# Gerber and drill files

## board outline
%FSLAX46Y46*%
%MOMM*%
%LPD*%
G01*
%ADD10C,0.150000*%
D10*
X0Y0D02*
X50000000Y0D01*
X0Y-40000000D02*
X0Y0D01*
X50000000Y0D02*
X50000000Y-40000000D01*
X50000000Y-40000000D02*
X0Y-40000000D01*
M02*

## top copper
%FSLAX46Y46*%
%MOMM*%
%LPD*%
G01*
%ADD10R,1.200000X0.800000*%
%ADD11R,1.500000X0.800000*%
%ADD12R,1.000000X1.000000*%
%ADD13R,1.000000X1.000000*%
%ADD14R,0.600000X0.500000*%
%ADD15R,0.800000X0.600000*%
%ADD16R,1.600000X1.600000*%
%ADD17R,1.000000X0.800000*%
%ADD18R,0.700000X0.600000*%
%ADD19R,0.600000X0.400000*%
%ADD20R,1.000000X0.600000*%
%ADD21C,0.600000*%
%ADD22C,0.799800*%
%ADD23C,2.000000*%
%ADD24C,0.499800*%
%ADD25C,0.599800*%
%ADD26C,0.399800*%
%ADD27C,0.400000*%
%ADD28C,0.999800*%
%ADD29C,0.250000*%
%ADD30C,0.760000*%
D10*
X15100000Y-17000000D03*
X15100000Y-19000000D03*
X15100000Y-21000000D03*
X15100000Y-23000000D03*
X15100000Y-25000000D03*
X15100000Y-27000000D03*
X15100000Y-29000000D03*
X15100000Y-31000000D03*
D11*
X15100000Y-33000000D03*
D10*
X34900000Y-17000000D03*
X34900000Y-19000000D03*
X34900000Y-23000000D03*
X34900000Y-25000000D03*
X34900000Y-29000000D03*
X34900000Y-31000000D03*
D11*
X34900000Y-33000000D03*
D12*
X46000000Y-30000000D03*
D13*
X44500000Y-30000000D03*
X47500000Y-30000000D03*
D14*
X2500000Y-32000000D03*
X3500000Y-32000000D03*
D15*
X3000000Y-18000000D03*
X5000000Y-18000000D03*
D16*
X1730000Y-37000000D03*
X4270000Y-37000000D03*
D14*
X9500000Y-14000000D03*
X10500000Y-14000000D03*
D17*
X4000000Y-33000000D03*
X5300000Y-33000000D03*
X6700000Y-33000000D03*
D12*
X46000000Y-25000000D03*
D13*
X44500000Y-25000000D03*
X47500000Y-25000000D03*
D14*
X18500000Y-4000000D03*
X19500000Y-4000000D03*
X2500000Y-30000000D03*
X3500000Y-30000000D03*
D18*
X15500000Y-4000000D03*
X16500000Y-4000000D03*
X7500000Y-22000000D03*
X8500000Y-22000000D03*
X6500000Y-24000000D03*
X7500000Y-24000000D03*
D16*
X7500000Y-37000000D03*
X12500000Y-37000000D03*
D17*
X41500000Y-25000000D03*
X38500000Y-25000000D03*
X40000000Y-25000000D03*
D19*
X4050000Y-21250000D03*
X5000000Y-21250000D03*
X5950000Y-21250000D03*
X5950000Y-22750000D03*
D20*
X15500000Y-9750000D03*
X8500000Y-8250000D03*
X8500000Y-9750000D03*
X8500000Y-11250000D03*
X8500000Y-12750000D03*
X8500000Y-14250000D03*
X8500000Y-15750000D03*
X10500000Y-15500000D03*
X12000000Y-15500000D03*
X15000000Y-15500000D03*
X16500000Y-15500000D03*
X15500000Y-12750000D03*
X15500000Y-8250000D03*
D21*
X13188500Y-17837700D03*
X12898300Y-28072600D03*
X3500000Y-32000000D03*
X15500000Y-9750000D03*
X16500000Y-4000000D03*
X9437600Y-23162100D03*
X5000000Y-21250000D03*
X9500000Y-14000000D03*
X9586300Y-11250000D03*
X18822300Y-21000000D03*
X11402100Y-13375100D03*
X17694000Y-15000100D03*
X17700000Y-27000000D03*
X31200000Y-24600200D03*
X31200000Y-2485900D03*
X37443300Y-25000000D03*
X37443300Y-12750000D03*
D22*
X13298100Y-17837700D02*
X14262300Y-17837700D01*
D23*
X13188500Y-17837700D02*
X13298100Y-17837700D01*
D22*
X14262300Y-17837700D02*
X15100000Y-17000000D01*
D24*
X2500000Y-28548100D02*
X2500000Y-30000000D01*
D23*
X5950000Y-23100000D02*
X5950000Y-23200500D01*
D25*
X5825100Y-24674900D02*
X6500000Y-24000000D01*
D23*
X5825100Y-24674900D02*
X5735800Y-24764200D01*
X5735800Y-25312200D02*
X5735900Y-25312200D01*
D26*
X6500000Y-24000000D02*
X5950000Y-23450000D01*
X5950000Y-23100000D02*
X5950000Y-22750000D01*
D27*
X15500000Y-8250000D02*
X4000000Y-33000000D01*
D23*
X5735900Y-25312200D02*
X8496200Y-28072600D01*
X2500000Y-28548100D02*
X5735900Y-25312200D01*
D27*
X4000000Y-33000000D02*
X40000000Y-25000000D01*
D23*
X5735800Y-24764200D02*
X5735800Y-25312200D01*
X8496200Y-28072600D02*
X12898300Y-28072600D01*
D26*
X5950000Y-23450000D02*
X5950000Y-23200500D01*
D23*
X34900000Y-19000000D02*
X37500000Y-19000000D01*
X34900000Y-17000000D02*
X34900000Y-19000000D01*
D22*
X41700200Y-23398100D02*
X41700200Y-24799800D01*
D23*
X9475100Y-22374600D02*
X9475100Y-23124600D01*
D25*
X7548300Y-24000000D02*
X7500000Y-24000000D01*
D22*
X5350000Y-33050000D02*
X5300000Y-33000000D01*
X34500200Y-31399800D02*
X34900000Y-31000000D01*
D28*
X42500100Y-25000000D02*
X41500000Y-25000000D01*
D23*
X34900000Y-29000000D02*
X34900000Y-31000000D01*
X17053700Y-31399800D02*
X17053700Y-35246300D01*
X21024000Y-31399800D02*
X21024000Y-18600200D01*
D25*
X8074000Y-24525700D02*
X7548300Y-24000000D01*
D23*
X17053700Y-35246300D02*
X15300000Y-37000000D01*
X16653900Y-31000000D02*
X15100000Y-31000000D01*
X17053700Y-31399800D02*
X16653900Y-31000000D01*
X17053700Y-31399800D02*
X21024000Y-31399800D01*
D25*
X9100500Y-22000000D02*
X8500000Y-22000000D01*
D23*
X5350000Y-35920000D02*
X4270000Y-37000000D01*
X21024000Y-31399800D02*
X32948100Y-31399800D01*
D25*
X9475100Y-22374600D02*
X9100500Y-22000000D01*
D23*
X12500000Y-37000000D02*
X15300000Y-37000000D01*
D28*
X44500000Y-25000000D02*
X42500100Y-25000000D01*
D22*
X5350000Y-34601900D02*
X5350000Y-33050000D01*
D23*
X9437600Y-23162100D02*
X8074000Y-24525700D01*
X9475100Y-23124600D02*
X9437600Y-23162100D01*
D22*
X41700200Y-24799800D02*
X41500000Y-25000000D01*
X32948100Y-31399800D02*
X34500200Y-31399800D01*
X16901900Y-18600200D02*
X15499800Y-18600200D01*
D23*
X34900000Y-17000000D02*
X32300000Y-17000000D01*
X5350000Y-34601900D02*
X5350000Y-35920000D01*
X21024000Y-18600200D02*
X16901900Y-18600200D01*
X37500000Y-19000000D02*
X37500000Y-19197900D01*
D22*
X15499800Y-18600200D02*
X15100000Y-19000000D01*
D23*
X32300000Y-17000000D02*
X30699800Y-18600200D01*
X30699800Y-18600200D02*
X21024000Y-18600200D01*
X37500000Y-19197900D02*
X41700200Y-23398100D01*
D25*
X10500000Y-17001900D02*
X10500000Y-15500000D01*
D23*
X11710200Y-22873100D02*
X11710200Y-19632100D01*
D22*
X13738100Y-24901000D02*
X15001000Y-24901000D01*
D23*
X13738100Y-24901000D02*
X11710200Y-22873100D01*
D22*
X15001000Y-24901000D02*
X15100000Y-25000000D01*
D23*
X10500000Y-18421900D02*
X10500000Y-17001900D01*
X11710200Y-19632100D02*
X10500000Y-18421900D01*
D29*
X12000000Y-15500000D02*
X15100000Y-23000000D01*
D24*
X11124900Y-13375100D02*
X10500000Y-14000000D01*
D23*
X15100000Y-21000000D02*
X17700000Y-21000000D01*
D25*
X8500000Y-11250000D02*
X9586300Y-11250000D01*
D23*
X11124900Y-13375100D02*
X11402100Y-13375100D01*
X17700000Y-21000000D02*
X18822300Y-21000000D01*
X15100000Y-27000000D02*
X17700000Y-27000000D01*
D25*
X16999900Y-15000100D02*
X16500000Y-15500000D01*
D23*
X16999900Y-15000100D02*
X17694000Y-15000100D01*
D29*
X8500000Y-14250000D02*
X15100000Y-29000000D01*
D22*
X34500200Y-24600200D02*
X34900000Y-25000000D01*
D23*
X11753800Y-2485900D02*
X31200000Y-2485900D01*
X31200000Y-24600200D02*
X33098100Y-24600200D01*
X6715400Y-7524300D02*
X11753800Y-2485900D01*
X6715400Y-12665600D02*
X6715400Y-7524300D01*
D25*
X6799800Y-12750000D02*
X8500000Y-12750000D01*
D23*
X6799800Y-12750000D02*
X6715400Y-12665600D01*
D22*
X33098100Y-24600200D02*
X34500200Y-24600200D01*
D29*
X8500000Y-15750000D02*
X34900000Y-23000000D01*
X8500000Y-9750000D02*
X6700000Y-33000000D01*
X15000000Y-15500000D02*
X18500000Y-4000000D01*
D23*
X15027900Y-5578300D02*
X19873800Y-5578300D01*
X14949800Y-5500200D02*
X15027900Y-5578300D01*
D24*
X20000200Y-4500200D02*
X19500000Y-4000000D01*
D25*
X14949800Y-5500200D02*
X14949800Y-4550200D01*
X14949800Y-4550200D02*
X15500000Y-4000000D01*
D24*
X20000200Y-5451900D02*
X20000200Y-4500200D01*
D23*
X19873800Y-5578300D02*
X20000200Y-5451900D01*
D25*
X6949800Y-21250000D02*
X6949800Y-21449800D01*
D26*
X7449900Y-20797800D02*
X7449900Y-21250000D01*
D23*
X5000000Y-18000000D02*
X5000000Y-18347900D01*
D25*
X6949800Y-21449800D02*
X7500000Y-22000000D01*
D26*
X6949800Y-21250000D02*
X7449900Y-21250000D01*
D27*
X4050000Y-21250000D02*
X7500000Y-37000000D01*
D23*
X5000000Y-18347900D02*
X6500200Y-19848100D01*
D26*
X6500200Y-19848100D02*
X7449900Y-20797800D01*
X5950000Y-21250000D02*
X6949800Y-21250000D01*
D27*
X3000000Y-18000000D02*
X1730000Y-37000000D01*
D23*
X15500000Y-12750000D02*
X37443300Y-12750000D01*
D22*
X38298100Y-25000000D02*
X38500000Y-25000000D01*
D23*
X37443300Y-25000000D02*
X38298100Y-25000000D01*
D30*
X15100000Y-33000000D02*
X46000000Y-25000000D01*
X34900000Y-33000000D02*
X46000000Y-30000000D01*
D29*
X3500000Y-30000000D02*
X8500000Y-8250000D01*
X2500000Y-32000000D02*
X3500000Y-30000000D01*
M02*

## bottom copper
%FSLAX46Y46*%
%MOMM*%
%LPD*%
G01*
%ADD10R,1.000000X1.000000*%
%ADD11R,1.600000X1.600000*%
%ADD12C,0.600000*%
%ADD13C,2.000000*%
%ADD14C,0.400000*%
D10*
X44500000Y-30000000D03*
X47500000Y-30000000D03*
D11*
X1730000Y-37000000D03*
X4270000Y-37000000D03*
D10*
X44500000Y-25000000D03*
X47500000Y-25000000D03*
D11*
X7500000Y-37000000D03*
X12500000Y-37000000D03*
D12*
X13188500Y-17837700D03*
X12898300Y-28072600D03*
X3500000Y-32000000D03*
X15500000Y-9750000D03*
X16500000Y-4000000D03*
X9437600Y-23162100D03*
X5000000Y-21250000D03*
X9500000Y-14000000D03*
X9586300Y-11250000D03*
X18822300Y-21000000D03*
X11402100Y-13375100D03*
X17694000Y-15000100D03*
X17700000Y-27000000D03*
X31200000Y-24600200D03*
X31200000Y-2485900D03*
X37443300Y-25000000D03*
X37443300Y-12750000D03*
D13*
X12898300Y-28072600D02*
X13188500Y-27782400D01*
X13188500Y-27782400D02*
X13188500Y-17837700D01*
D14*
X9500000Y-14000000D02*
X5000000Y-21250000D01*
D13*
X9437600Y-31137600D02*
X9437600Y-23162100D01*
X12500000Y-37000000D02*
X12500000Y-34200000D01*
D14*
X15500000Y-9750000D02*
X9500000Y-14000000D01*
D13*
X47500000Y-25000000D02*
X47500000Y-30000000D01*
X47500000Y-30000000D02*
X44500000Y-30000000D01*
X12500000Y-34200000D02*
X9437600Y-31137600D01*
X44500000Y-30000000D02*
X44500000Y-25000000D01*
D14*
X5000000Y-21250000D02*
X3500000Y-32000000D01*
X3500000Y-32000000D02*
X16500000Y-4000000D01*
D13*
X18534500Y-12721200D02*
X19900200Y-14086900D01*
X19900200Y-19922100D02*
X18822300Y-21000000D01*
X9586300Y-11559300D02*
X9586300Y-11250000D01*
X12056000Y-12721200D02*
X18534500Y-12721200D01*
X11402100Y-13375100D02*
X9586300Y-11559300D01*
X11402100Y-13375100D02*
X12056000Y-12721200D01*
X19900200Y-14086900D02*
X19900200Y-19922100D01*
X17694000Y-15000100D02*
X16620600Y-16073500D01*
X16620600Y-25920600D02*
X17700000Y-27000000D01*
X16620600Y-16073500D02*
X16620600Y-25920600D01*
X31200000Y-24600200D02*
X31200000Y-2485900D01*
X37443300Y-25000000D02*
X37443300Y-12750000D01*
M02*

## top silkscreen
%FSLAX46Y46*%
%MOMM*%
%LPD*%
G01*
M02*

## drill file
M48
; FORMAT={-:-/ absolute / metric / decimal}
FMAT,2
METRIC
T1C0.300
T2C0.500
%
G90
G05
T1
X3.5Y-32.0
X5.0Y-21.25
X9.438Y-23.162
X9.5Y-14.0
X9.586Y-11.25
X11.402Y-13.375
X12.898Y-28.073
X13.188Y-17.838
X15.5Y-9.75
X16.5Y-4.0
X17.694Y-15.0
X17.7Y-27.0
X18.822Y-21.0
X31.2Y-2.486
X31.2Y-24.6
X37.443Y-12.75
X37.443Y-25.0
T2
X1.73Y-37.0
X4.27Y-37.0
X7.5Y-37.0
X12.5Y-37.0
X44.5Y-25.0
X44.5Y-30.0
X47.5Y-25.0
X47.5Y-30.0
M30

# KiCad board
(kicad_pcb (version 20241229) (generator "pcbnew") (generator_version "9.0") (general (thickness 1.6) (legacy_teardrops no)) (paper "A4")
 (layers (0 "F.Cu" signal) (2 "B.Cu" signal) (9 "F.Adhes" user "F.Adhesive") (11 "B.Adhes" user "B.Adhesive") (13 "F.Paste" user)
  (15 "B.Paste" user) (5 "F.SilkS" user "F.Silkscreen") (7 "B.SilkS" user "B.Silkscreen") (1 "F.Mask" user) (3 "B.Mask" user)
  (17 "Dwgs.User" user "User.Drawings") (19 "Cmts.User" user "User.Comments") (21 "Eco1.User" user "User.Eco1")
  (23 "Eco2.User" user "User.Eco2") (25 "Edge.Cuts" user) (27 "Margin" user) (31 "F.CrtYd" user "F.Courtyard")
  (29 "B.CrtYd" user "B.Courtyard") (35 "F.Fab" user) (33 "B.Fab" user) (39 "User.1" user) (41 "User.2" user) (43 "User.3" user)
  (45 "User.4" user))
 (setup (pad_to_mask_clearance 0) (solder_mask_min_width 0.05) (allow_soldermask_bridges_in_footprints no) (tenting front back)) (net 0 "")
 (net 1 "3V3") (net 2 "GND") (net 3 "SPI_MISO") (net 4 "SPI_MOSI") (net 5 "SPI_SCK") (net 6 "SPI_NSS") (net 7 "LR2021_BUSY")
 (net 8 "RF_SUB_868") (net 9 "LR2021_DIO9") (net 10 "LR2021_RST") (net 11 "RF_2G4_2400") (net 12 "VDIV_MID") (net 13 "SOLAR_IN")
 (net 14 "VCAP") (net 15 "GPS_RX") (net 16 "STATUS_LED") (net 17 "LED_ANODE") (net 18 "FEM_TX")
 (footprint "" (layer "F.Cu") (at 25 25)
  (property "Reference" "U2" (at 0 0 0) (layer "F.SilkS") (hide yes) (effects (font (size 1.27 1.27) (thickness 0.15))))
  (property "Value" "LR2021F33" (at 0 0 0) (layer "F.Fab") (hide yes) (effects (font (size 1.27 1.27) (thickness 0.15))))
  (pad "1" smd rect (at -9.9 -8) (size 1.2 0.8) (layers "F.Cu" "F.Mask") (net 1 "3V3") (thermal_bridge_angle 45))
  (pad "2" smd rect (at -9.9 -6) (size 1.2 0.8) (layers "F.Cu" "F.Mask") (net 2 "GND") (thermal_bridge_angle 45))
  (pad "3" smd rect (at -9.9 -4) (size 1.2 0.8) (layers "F.Cu" "F.Mask") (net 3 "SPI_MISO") (thermal_bridge_angle 45))
  (pad "4" smd rect (at -9.9 -2) (size 1.2 0.8) (layers "F.Cu" "F.Mask") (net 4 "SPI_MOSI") (thermal_bridge_angle 45))
  (pad "5" smd rect (at -9.9 0) (size 1.2 0.8) (layers "F.Cu" "F.Mask") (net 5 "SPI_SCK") (thermal_bridge_angle 45))
  (pad "6" smd rect (at -9.9 2) (size 1.2 0.8) (layers "F.Cu" "F.Mask") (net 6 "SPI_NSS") (thermal_bridge_angle 45))
  (pad "7" smd rect (at -9.9 4) (size 1.2 0.8) (layers "F.Cu" "F.Mask") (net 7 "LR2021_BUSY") (thermal_bridge_angle 45))
  (pad "8" smd rect (at -9.9 6) (size 1.2 0.8) (layers "F.Cu" "F.Mask") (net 2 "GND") (thermal_bridge_angle 45))
  (pad "9" smd rect (at -9.9 8) (size 1.5 0.8) (layers "F.Cu" "F.Mask") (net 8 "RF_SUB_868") (thermal_bridge_angle 45))
  (pad "10" smd rect (at 9.9 -8) (size 1.2 0.8) (layers "F.Cu" "F.Mask") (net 2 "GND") (thermal_bridge_angle 45))
  (pad "11" smd rect (at 9.9 -6) (size 1.2 0.8) (layers "F.Cu" "F.Mask") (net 2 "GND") (thermal_bridge_angle 45))
  (pad "13" smd rect (at 9.9 -2) (size 1.2 0.8) (layers "F.Cu" "F.Mask") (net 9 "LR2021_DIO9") (thermal_bridge_angle 45))
  (pad "14" smd rect (at 9.9 0) (size 1.2 0.8) (layers "F.Cu" "F.Mask") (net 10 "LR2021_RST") (thermal_bridge_angle 45))
  (pad "16" smd rect (at 9.9 4) (size 1.2 0.8) (layers "F.Cu" "F.Mask") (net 2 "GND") (thermal_bridge_angle 45))
  (pad "17" smd rect (at 9.9 6) (size 1.2 0.8) (layers "F.Cu" "F.Mask") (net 2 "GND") (thermal_bridge_angle 45))
  (pad "18" smd rect (at 9.9 8) (size 1.5 0.8) (layers "F.Cu" "F.Mask") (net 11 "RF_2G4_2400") (thermal_bridge_angle 45)))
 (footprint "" (layer "F.Cu") (at 46 30)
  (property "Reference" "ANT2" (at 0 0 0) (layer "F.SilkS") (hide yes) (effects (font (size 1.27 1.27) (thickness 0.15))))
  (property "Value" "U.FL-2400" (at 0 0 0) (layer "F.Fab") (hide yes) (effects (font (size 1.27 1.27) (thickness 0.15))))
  (pad "1" smd rect (at 0 0) (size 1 1) (layers "F.Cu" "F.Mask") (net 11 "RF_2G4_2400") (thermal_bridge_angle 45))
  (pad "2" thru_hole rect (at -1.5 0) (size 1 1) (drill 0.5) (layers "*.Cu" "*.Mask") (remove_unused_layers no) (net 2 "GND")
   (thermal_bridge_angle 45))
  (pad "3" thru_hole rect (at 1.5 0) (size 1 1) (drill 0.5) (layers "*.Cu" "*.Mask") (remove_unused_layers no) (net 2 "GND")
   (thermal_bridge_angle 45)))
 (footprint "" (layer "F.Cu") (at 3 32)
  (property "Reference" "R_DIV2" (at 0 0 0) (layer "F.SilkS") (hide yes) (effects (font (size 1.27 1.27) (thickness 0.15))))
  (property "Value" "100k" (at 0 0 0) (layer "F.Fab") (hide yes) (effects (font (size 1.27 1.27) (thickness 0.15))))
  (pad "1" smd rect (at -0.5 0) (size 0.6 0.5) (layers "F.Cu" "F.Mask") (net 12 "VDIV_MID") (thermal_bridge_angle 45))
  (pad "2" smd rect (at 0.5 0) (size 0.6 0.5) (layers "F.Cu" "F.Mask") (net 2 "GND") (thermal_bridge_angle 45)))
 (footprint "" (layer "F.Cu") (at 4 18)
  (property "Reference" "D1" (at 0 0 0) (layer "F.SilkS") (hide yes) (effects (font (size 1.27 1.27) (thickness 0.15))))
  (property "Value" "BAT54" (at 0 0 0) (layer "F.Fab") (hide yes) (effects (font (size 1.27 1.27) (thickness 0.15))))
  (pad "A" smd rect (at -1 0) (size 0.8 0.6) (layers "F.Cu" "F.Mask") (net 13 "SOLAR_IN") (thermal_bridge_angle 45))
  (pad "K" smd rect (at 1 0) (size 0.8 0.6) (layers "F.Cu" "F.Mask") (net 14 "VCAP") (thermal_bridge_angle 45)))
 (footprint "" (layer "F.Cu") (at 3 37)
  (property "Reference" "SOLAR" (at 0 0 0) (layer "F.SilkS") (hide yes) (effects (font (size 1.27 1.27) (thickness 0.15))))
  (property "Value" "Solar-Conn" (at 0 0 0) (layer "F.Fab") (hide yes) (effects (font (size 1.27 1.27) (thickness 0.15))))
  (pad "1" thru_hole rect (at -1.27 0) (size 1.6 1.6) (drill 0.5) (layers "*.Cu" "*.Mask") (remove_unused_layers no) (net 13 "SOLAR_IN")
   (thermal_bridge_angle 45))
  (pad "2" thru_hole rect (at 1.27 0) (size 1.6 1.6) (drill 0.5) (layers "*.Cu" "*.Mask") (remove_unused_layers no) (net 2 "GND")
   (thermal_bridge_angle 45)))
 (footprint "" (layer "F.Cu") (at 10 14)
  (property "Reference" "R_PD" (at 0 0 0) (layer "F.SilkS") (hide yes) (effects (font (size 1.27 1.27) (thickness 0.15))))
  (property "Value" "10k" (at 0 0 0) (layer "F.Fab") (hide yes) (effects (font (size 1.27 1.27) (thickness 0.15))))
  (pad "1" smd rect (at -0.5 0) (size 0.6 0.5) (layers "F.Cu" "F.Mask") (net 2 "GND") (thermal_bridge_angle 45))
  (pad "2" smd rect (at 0.5 0) (size 0.6 0.5) (layers "F.Cu" "F.Mask") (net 3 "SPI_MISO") (thermal_bridge_angle 45)))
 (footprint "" (layer "F.Cu") (at 6 33)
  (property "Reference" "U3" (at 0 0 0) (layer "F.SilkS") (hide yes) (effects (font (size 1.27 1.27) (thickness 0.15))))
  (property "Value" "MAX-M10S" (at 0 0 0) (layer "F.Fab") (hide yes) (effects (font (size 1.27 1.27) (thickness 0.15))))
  (pad "1" smd rect (at -2 0) (size 1 0.8) (layers "F.Cu" "F.Mask") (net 1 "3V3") (thermal_bridge_angle 45))
  (pad "2" smd rect (at -0.7 0) (size 1 0.8) (layers "F.Cu" "F.Mask") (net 2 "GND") (thermal_bridge_angle 45))
  (pad "3" smd rect (at 0.7 0) (size 1 0.8) (layers "F.Cu" "F.Mask") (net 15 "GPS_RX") (thermal_bridge_angle 45)))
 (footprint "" (layer "F.Cu") (at 46 25)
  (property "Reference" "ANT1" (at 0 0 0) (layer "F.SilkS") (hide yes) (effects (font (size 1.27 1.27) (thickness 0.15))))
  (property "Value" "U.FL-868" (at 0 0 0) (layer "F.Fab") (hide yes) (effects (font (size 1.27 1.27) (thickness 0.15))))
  (pad "1" smd rect (at 0 0) (size 1 1) (layers "F.Cu" "F.Mask") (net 8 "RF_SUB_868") (thermal_bridge_angle 45))
  (pad "2" thru_hole rect (at -1.5 0) (size 1 1) (drill 0.5) (layers "*.Cu" "*.Mask") (remove_unused_layers no) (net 2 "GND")
   (thermal_bridge_angle 45))
  (pad "3" thru_hole rect (at 1.5 0) (size 1 1) (drill 0.5) (layers "*.Cu" "*.Mask") (remove_unused_layers no) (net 2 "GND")
   (thermal_bridge_angle 45)))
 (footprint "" (layer "F.Cu") (at 19 4)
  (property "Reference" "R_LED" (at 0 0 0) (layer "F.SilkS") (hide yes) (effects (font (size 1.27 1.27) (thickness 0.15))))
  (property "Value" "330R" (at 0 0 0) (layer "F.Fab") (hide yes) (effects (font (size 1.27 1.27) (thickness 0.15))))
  (pad "1" smd rect (at -0.5 0) (size 0.6 0.5) (layers "F.Cu" "F.Mask") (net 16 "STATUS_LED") (thermal_bridge_angle 45))
  (pad "2" smd rect (at 0.5 0) (size 0.6 0.5) (layers "F.Cu" "F.Mask") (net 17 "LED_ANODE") (thermal_bridge_angle 45)))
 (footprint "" (layer "F.Cu") (at 3 30)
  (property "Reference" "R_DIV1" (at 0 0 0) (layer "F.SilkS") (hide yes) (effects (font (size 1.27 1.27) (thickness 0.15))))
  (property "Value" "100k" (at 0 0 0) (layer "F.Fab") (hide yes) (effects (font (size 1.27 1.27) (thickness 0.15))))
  (pad "1" smd rect (at -0.5 0) (size 0.6 0.5) (layers "F.Cu" "F.Mask") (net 1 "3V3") (thermal_bridge_angle 45))
  (pad "2" smd rect (at 0.5 0) (size 0.6 0.5) (layers "F.Cu" "F.Mask") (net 12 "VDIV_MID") (thermal_bridge_angle 45)))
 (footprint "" (layer "F.Cu") (at 16 4)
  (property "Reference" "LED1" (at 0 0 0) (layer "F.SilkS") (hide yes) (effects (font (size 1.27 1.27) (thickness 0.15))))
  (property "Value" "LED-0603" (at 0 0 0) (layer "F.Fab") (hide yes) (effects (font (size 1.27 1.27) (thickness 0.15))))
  (pad "A" smd rect (at -0.5 0) (size 0.7 0.6) (layers "F.Cu" "F.Mask") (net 17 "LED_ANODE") (thermal_bridge_angle 45))
  (pad "K" smd rect (at 0.5 0) (size 0.7 0.6) (layers "F.Cu" "F.Mask") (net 2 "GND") (thermal_bridge_angle 45)))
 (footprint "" (layer "F.Cu") (at 8 22)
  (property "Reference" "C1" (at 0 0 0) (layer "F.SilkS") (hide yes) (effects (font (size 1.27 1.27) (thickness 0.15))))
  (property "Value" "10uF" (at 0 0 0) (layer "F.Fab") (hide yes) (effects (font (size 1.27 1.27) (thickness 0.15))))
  (pad "1" smd rect (at -0.5 0) (size 0.7 0.6) (layers "F.Cu" "F.Mask") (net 14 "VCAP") (thermal_bridge_angle 45))
  (pad "2" smd rect (at 0.5 0) (size 0.7 0.6) (layers "F.Cu" "F.Mask") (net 2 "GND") (thermal_bridge_angle 45)))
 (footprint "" (layer "F.Cu") (at 7 24)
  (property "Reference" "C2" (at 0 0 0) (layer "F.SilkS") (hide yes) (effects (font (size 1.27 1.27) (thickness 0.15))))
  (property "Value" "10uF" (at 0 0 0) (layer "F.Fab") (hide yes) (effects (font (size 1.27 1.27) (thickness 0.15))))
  (pad "1" smd rect (at -0.5 0) (size 0.7 0.6) (layers "F.Cu" "F.Mask") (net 1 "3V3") (thermal_bridge_angle 45))
  (pad "2" smd rect (at 0.5 0) (size 0.7 0.6) (layers "F.Cu" "F.Mask") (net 2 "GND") (thermal_bridge_angle 45)))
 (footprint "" (layer "F.Cu") (at 10 37)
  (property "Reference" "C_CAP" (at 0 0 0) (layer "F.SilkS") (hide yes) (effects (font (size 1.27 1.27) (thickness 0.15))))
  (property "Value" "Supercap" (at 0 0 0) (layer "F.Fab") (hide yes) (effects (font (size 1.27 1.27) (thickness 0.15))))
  (pad "1" thru_hole rect (at -2.5 0) (size 1.6 1.6) (drill 0.5) (layers "*.Cu" "*.Mask") (remove_unused_layers no) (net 14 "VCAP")
   (thermal_bridge_angle 45))
  (pad "2" thru_hole rect (at 2.5 0) (size 1.6 1.6) (drill 0.5) (layers "*.Cu" "*.Mask") (remove_unused_layers no) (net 2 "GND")
   (thermal_bridge_angle 45)))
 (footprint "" (layer "F.Cu") (at 40 25)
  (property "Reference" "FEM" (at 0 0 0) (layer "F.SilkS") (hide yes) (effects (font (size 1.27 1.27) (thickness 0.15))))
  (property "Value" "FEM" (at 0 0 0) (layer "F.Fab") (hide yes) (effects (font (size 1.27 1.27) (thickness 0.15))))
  (pad "GND" smd rect (at 1.5 0) (size 1 0.8) (layers "F.Cu" "F.Mask") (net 2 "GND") (thermal_bridge_angle 45))
  (pad "TX" smd rect (at -1.5 0) (size 1 0.8) (layers "F.Cu" "F.Mask") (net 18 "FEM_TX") (thermal_bridge_angle 45))
  (pad "VCC" smd rect (at 0 0) (size 1 0.8) (layers "F.Cu" "F.Mask") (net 1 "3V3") (thermal_bridge_angle 45)))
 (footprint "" (layer "F.Cu") (at 5 22)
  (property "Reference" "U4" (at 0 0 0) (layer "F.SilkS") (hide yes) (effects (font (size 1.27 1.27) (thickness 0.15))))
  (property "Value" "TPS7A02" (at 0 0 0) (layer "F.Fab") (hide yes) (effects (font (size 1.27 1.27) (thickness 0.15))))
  (pad "1" smd rect (at -0.95 -0.75) (size 0.6 0.4) (layers "F.Cu" "F.Mask") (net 14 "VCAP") (thermal_bridge_angle 45))
  (pad "2" smd rect (at 0 -0.75) (size 0.6 0.4) (layers "F.Cu" "F.Mask") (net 2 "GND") (thermal_bridge_angle 45))
  (pad "3" smd rect (at 0.95 -0.75) (size 0.6 0.4) (layers "F.Cu" "F.Mask") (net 14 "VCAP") (thermal_bridge_angle 45))
  (pad "4" smd rect (at 0.95 0.75) (size 0.6 0.4) (layers "F.Cu" "F.Mask") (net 1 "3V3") (thermal_bridge_angle 45)))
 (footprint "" (layer "F.Cu") (at 12 12)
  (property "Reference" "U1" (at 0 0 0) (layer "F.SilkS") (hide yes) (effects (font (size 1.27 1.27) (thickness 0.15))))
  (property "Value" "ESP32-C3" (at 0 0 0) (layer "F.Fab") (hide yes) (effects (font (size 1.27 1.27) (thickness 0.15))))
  (pad "GND" smd rect (at 3.5 -2.25) (size 1 0.6) (layers "F.Cu" "F.Mask") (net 2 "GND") (thermal_bridge_angle 45))
  (pad "GPIO0" smd rect (at -3.5 -3.75) (size 1 0.6) (layers "F.Cu" "F.Mask") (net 12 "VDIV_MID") (thermal_bridge_angle 45))
  (pad "GPIO1" smd rect (at -3.5 -2.25) (size 1 0.6) (layers "F.Cu" "F.Mask") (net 15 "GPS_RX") (thermal_bridge_angle 45))
  (pad "GPIO2" smd rect (at -3.5 -0.75) (size 1 0.6) (layers "F.Cu" "F.Mask") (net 3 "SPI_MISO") (thermal_bridge_angle 45))
  (pad "GPIO3" smd rect (at -3.5 0.75) (size 1 0.6) (layers "F.Cu" "F.Mask") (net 10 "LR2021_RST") (thermal_bridge_angle 45))
  (pad "GPIO4" smd rect (at -3.5 2.25) (size 1 0.6) (layers "F.Cu" "F.Mask") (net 7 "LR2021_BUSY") (thermal_bridge_angle 45))
  (pad "GPIO5" smd rect (at -3.5 3.75) (size 1 0.6) (layers "F.Cu" "F.Mask") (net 9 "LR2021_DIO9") (thermal_bridge_angle 45))
  (pad "GPIO6" smd rect (at -1.5 3.5) (size 1 0.6) (layers "F.Cu" "F.Mask") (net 5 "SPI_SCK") (thermal_bridge_angle 45))
  (pad "GPIO7" smd rect (at 0 3.5) (size 1 0.6) (layers "F.Cu" "F.Mask") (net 4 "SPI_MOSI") (thermal_bridge_angle 45))
  (pad "GPIO9" smd rect (at 3 3.5) (size 1 0.6) (layers "F.Cu" "F.Mask") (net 16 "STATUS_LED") (thermal_bridge_angle 45))
  (pad "GPIO10" smd rect (at 4.5 3.5) (size 1 0.6) (layers "F.Cu" "F.Mask") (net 6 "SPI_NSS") (thermal_bridge_angle 45))
  (pad "GPIO19" smd rect (at 3.5 0.75) (size 1 0.6) (layers "F.Cu" "F.Mask") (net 18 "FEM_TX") (thermal_bridge_angle 45))
  (pad "VCC" smd rect (at 3.5 -3.75) (size 1 0.6) (layers "F.Cu" "F.Mask") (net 1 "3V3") (thermal_bridge_angle 45)))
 (gr_line (start 0 0) (end 50 0) (stroke (width 0.15) (type default)) (layer "Edge.Cuts"))
 (gr_line (start 0 40) (end 0 0) (stroke (width 0.15) (type default)) (layer "Edge.Cuts"))
 (gr_line (start 50 0) (end 50 40) (stroke (width 0.15) (type default)) (layer "Edge.Cuts"))
 (gr_line (start 50 40) (end 0 40) (stroke (width 0.15) (type default)) (layer "Edge.Cuts"))
 (segment (start 13.2981 17.8377) (end 14.2623 17.8377) (width 0.7998) (layer "F.Cu") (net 1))
 (segment (start 13.1885 17.8377) (end 13.2981 17.8377) (width 2) (layer "F.Cu") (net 1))
 (segment (start 14.2623 17.8377) (end 15.1 17) (width 0.7998) (layer "F.Cu") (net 1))
 (segment (start 2.5 28.5481) (end 2.5 30) (width 0.4998) (layer "F.Cu") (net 1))
 (segment (start 5.95 23.1) (end 5.95 23.2005) (width 2) (layer "F.Cu") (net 1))
 (segment (start 5.8251 24.6749) (end 6.5 24) (width 0.5998) (layer "F.Cu") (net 1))
 (segment (start 5.8251 24.6749) (end 5.7358 24.7642) (width 2) (layer "F.Cu") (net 1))
 (segment (start 5.7358 25.3122) (end 5.7359 25.3122) (width 2) (layer "F.Cu") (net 1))
 (segment (start 6.5 24) (end 5.95 23.45) (width 0.3998) (layer "F.Cu") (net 1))
 (segment (start 5.95 23.1) (end 5.95 22.75) (width 0.3998) (layer "F.Cu") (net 1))
 (segment (start 15.5 8.25) (end 4 33) (width 0.4) (layer "F.Cu") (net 1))
 (segment (start 5.7359 25.3122) (end 8.4962 28.0726) (width 2) (layer "F.Cu") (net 1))
 (segment (start 2.5 28.5481) (end 5.7359 25.3122) (width 2) (layer "F.Cu") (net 1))
 (segment (start 4 33) (end 40 25) (width 0.4) (layer "F.Cu") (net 1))
 (segment (start 5.7358 24.7642) (end 5.7358 25.3122) (width 2) (layer "F.Cu") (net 1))
 (segment (start 8.4962 28.0726) (end 12.8983 28.0726) (width 2) (layer "F.Cu") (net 1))
 (segment (start 5.95 23.45) (end 5.95 23.2005) (width 0.3998) (layer "F.Cu") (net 1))
 (via (at 13.1885 17.8377) (size 0.6) (drill 0.3) (layers "F.Cu" "B.Cu") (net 1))
 (via (at 12.8983 28.0726) (size 0.6) (drill 0.3) (layers "F.Cu" "B.Cu") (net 1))
 (segment (start 12.8983 28.0726) (end 13.1885 27.7824) (width 2) (layer "B.Cu") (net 1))
 (segment (start 13.1885 27.7824) (end 13.1885 17.8377) (width 2) (layer "B.Cu") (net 1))
 (segment (start 34.9 19) (end 37.5 19) (width 2) (layer "F.Cu") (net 2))
 (segment (start 34.9 17) (end 34.9 19) (width 2) (layer "F.Cu") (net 2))
 (segment (start 41.7002 23.3981) (end 41.7002 24.7998) (width 0.7998) (layer "F.Cu") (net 2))
 (segment (start 9.4751 22.3746) (end 9.4751 23.1246) (width 2) (layer "F.Cu") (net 2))
 (segment (start 7.5483 24) (end 7.5 24) (width 0.5998) (layer "F.Cu") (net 2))
 (segment (start 5.35 33.05) (end 5.3 33) (width 0.7998) (layer "F.Cu") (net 2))
 (segment (start 34.5002 31.3998) (end 34.9 31) (width 0.7998) (layer "F.Cu") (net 2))
 (segment (start 42.5001 25) (end 41.5 25) (width 0.9998) (layer "F.Cu") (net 2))
 (segment (start 34.9 29) (end 34.9 31) (width 2) (layer "F.Cu") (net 2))
 (segment (start 17.0537 31.3998) (end 17.0537 35.2463) (width 2) (layer "F.Cu") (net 2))
 (segment (start 21.024 31.3998) (end 21.024 18.6002) (width 2) (layer "F.Cu") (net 2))
 (segment (start 8.074 24.5257) (end 7.5483 24) (width 0.5998) (layer "F.Cu") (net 2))
 (segment (start 17.0537 35.2463) (end 15.3 37) (width 2) (layer "F.Cu") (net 2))
 (segment (start 16.6539 31) (end 15.1 31) (width 2) (layer "F.Cu") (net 2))
 (segment (start 17.0537 31.3998) (end 16.6539 31) (width 2) (layer "F.Cu") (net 2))
 (segment (start 17.0537 31.3998) (end 21.024 31.3998) (width 2) (layer "F.Cu") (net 2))
 (segment (start 9.1005 22) (end 8.5 22) (width 0.5998) (layer "F.Cu") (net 2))
 (segment (start 5.35 35.92) (end 4.27 37) (width 2) (layer "F.Cu") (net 2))
 (segment (start 21.024 31.3998) (end 32.9481 31.3998) (width 2) (layer "F.Cu") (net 2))
 (segment (start 9.4751 22.3746) (end 9.1005 22) (width 0.5998) (layer "F.Cu") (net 2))
 (segment (start 12.5 37) (end 15.3 37) (width 2) (layer "F.Cu") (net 2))
 (segment (start 44.5 25) (end 42.5001 25) (width 0.9998) (layer "F.Cu") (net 2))
 (segment (start 5.35 34.6019) (end 5.35 33.05) (width 0.7998) (layer "F.Cu") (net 2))
 (segment (start 9.4376 23.1621) (end 8.074 24.5257) (width 2) (layer "F.Cu") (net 2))
 (segment (start 9.4751 23.1246) (end 9.4376 23.1621) (width 2) (layer "F.Cu") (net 2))
 (segment (start 41.7002 24.7998) (end 41.5 25) (width 0.7998) (layer "F.Cu") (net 2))
 (segment (start 32.9481 31.3998) (end 34.5002 31.3998) (width 0.7998) (layer "F.Cu") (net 2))
 (segment (start 16.9019 18.6002) (end 15.4998 18.6002) (width 0.7998) (layer "F.Cu") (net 2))
 (segment (start 34.9 17) (end 32.3 17) (width 2) (layer "F.Cu") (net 2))
 (segment (start 5.35 34.6019) (end 5.35 35.92) (width 2) (layer "F.Cu") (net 2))
 (segment (start 21.024 18.6002) (end 16.9019 18.6002) (width 2) (layer "F.Cu") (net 2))
 (segment (start 37.5 19) (end 37.5 19.1979) (width 2) (layer "F.Cu") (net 2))
 (segment (start 15.4998 18.6002) (end 15.1 19) (width 0.7998) (layer "F.Cu") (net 2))
 (segment (start 32.3 17) (end 30.6998 18.6002) (width 2) (layer "F.Cu") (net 2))
 (segment (start 30.6998 18.6002) (end 21.024 18.6002) (width 2) (layer "F.Cu") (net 2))
 (segment (start 37.5 19.1979) (end 41.7002 23.3981) (width 2) (layer "F.Cu") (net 2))
 (via (at 3.5 32) (size 0.6) (drill 0.3) (layers "F.Cu" "B.Cu") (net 2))
 (via (at 15.5 9.75) (size 0.6) (drill 0.3) (layers "F.Cu" "B.Cu") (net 2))
 (via (at 16.5 4) (size 0.6) (drill 0.3) (layers "F.Cu" "B.Cu") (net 2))
 (via (at 9.4376 23.1621) (size 0.6) (drill 0.3) (layers "F.Cu" "B.Cu") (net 2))
 (via (at 5 21.25) (size 0.6) (drill 0.3) (layers "F.Cu" "B.Cu") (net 2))
 (via (at 9.5 14) (size 0.6) (drill 0.3) (layers "F.Cu" "B.Cu") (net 2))
 (segment (start 9.5 14) (end 5 21.25) (width 0.4) (layer "B.Cu") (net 2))
 (segment (start 9.4376 31.1376) (end 9.4376 23.1621) (width 2) (layer "B.Cu") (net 2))
 (segment (start 12.5 37) (end 12.5 34.2) (width 2) (layer "B.Cu") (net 2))
 (segment (start 15.5 9.75) (end 9.5 14) (width 0.4) (layer "B.Cu") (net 2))
 (segment (start 47.5 25) (end 47.5 30) (width 2) (layer "B.Cu") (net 2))
 (segment (start 47.5 30) (end 44.5 30) (width 2) (layer "B.Cu") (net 2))
 (segment (start 12.5 34.2) (end 9.4376 31.1376) (width 2) (layer "B.Cu") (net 2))
 (segment (start 44.5 30) (end 44.5 25) (width 2) (layer "B.Cu") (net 2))
 (segment (start 5 21.25) (end 3.5 32) (width 0.4) (layer "B.Cu") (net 2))
 (segment (start 3.5 32) (end 16.5 4) (width 0.4) (layer "B.Cu") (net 2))
 (segment (start 10.5 17.0019) (end 10.5 15.5) (width 0.5998) (layer "F.Cu") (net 5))
 (segment (start 11.7102 22.8731) (end 11.7102 19.6321) (width 2) (layer "F.Cu") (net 5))
 (segment (start 13.7381 24.901) (end 15.001 24.901) (width 0.7998) (layer "F.Cu") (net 5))
 (segment (start 13.7381 24.901) (end 11.7102 22.8731) (width 2) (layer "F.Cu") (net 5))
 (segment (start 15.001 24.901) (end 15.1 25) (width 0.7998) (layer "F.Cu") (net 5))
 (segment (start 10.5 18.4219) (end 10.5 17.0019) (width 2) (layer "F.Cu") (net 5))
 (segment (start 11.7102 19.6321) (end 10.5 18.4219) (width 2) (layer "F.Cu") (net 5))
 (segment (start 12 15.5) (end 15.1 23) (width 0.25) (layer "F.Cu") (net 4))
 (segment (start 11.1249 13.3751) (end 10.5 14) (width 0.4998) (layer "F.Cu") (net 3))
 (segment (start 15.1 21) (end 17.7 21) (width 2) (layer "F.Cu") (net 3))
 (segment (start 8.5 11.25) (end 9.5863 11.25) (width 0.5998) (layer "F.Cu") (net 3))
 (segment (start 11.1249 13.3751) (end 11.4021 13.3751) (width 2) (layer "F.Cu") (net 3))
 (segment (start 17.7 21) (end 18.8223 21) (width 2) (layer "F.Cu") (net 3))
 (via (at 9.5863 11.25) (size 0.6) (drill 0.3) (layers "F.Cu" "B.Cu") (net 3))
 (via (at 18.8223 21) (size 0.6) (drill 0.3) (layers "F.Cu" "B.Cu") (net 3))
 (via (at 11.4021 13.3751) (size 0.6) (drill 0.3) (layers "F.Cu" "B.Cu") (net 3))
 (segment (start 18.5345 12.7212) (end 19.9002 14.0869) (width 2) (layer "B.Cu") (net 3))
 (segment (start 19.9002 19.9221) (end 18.8223 21) (width 2) (layer "B.Cu") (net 3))
 (segment (start 9.5863 11.5593) (end 9.5863 11.25) (width 2) (layer "B.Cu") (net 3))
 (segment (start 12.056 12.7212) (end 18.5345 12.7212) (width 2) (layer "B.Cu") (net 3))
 (segment (start 11.4021 13.3751) (end 9.5863 11.5593) (width 2) (layer "B.Cu") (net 3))
 (segment (start 11.4021 13.3751) (end 12.056 12.7212) (width 2) (layer "B.Cu") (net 3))
 (segment (start 19.9002 14.0869) (end 19.9002 19.9221) (width 2) (layer "B.Cu") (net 3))
 (segment (start 15.1 27) (end 17.7 27) (width 2) (layer "F.Cu") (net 6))
 (segment (start 16.9999 15.0001) (end 16.5 15.5) (width 0.5998) (layer "F.Cu") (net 6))
 (segment (start 16.9999 15.0001) (end 17.694 15.0001) (width 2) (layer "F.Cu") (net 6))
 (via (at 17.694 15.0001) (size 0.6) (drill 0.3) (layers "F.Cu" "B.Cu") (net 6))
 (via (at 17.7 27) (size 0.6) (drill 0.3) (layers "F.Cu" "B.Cu") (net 6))
 (segment (start 17.694 15.0001) (end 16.6206 16.0735) (width 2) (layer "B.Cu") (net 6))
 (segment (start 16.6206 25.9206) (end 17.7 27) (width 2) (layer "B.Cu") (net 6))
 (segment (start 16.6206 16.0735) (end 16.6206 25.9206) (width 2) (layer "B.Cu") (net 6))
 (segment (start 8.5 14.25) (end 15.1 29) (width 0.25) (layer "F.Cu") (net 7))
 (segment (start 34.5002 24.6002) (end 34.9 25) (width 0.7998) (layer "F.Cu") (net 10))
 (segment (start 11.7538 2.4859) (end 31.2 2.4859) (width 2) (layer "F.Cu") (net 10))
 (segment (start 31.2 24.6002) (end 33.0981 24.6002) (width 2) (layer "F.Cu") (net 10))
 (segment (start 6.7154 7.5243) (end 11.7538 2.4859) (width 2) (layer "F.Cu") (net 10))
 (segment (start 6.7154 12.6656) (end 6.7154 7.5243) (width 2) (layer "F.Cu") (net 10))
 (segment (start 6.7998 12.75) (end 8.5 12.75) (width 0.5998) (layer "F.Cu") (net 10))
 (segment (start 6.7998 12.75) (end 6.7154 12.6656) (width 2) (layer "F.Cu") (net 10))
 (segment (start 33.0981 24.6002) (end 34.5002 24.6002) (width 0.7998) (layer "F.Cu") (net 10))
 (via (at 31.2 24.6002) (size 0.6) (drill 0.3) (layers "F.Cu" "B.Cu") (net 10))
 (via (at 31.2 2.4859) (size 0.6) (drill 0.3) (layers "F.Cu" "B.Cu") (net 10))
 (segment (start 31.2 24.6002) (end 31.2 2.4859) (width 2) (layer "B.Cu") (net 10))
 (segment (start 8.5 15.75) (end 34.9 23) (width 0.25) (layer "F.Cu") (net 9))
 (segment (start 8.5 9.75) (end 6.7 33) (width 0.25) (layer "F.Cu") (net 15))
 (segment (start 15 15.5) (end 18.5 4) (width 0.25) (layer "F.Cu") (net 16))
 (segment (start 15.0279 5.5783) (end 19.8738 5.5783) (width 2) (layer "F.Cu") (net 17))
 (segment (start 14.9498 5.5002) (end 15.0279 5.5783) (width 2) (layer "F.Cu") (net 17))
 (segment (start 20.0002 4.5002) (end 19.5 4) (width 0.4998) (layer "F.Cu") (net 17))
 (segment (start 14.9498 5.5002) (end 14.9498 4.5502) (width 0.5998) (layer "F.Cu") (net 17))
 (segment (start 14.9498 4.5502) (end 15.5 4) (width 0.5998) (layer "F.Cu") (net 17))
 (segment (start 20.0002 5.4519) (end 20.0002 4.5002) (width 0.4998) (layer "F.Cu") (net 17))
 (segment (start 19.8738 5.5783) (end 20.0002 5.4519) (width 2) (layer "F.Cu") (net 17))
 (segment (start 6.9498 21.25) (end 6.9498 21.4498) (width 0.5998) (layer "F.Cu") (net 14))
 (segment (start 7.4499 20.7978) (end 7.4499 21.25) (width 0.3998) (layer "F.Cu") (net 14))
 (segment (start 5 18) (end 5 18.3479) (width 2) (layer "F.Cu") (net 14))
 (segment (start 6.9498 21.4498) (end 7.5 22) (width 0.5998) (layer "F.Cu") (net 14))
 (segment (start 6.9498 21.25) (end 7.4499 21.25) (width 0.3998) (layer "F.Cu") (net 14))
 (segment (start 4.05 21.25) (end 7.5 37) (width 0.4) (layer "F.Cu") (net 14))
 (segment (start 5 18.3479) (end 6.5002 19.8481) (width 2) (layer "F.Cu") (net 14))
 (segment (start 6.5002 19.8481) (end 7.4499 20.7978) (width 0.3998) (layer "F.Cu") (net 14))
 (segment (start 5.95 21.25) (end 6.9498 21.25) (width 0.3998) (layer "F.Cu") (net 14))
 (segment (start 3 18) (end 1.73 37) (width 0.4) (layer "F.Cu") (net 13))
 (segment (start 15.5 12.75) (end 37.4433 12.75) (width 2) (layer "F.Cu") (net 18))
 (segment (start 38.2981 25) (end 38.5 25) (width 0.7998) (layer "F.Cu") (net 18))
 (segment (start 37.4433 25) (end 38.2981 25) (width 2) (layer "F.Cu") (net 18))
 (via (at 37.4433 25) (size 0.6) (drill 0.3) (layers "F.Cu" "B.Cu") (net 18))
 (via (at 37.4433 12.75) (size 0.6) (drill 0.3) (layers "F.Cu" "B.Cu") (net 18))
 (segment (start 37.4433 25) (end 37.4433 12.75) (width 2) (layer "B.Cu") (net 18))
 (segment (start 15.1 33) (end 46 25) (width 0.76) (layer "F.Cu") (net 8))
 (segment (start 34.9 33) (end 46 30) (width 0.76) (layer "F.Cu") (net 11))
 (segment (start 3.5 30) (end 8.5 8.25) (width 0.25) (layer "F.Cu") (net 12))
 (segment (start 2.5 32) (end 3.5 30) (width 0.25) (layer "F.Cu") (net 12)))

